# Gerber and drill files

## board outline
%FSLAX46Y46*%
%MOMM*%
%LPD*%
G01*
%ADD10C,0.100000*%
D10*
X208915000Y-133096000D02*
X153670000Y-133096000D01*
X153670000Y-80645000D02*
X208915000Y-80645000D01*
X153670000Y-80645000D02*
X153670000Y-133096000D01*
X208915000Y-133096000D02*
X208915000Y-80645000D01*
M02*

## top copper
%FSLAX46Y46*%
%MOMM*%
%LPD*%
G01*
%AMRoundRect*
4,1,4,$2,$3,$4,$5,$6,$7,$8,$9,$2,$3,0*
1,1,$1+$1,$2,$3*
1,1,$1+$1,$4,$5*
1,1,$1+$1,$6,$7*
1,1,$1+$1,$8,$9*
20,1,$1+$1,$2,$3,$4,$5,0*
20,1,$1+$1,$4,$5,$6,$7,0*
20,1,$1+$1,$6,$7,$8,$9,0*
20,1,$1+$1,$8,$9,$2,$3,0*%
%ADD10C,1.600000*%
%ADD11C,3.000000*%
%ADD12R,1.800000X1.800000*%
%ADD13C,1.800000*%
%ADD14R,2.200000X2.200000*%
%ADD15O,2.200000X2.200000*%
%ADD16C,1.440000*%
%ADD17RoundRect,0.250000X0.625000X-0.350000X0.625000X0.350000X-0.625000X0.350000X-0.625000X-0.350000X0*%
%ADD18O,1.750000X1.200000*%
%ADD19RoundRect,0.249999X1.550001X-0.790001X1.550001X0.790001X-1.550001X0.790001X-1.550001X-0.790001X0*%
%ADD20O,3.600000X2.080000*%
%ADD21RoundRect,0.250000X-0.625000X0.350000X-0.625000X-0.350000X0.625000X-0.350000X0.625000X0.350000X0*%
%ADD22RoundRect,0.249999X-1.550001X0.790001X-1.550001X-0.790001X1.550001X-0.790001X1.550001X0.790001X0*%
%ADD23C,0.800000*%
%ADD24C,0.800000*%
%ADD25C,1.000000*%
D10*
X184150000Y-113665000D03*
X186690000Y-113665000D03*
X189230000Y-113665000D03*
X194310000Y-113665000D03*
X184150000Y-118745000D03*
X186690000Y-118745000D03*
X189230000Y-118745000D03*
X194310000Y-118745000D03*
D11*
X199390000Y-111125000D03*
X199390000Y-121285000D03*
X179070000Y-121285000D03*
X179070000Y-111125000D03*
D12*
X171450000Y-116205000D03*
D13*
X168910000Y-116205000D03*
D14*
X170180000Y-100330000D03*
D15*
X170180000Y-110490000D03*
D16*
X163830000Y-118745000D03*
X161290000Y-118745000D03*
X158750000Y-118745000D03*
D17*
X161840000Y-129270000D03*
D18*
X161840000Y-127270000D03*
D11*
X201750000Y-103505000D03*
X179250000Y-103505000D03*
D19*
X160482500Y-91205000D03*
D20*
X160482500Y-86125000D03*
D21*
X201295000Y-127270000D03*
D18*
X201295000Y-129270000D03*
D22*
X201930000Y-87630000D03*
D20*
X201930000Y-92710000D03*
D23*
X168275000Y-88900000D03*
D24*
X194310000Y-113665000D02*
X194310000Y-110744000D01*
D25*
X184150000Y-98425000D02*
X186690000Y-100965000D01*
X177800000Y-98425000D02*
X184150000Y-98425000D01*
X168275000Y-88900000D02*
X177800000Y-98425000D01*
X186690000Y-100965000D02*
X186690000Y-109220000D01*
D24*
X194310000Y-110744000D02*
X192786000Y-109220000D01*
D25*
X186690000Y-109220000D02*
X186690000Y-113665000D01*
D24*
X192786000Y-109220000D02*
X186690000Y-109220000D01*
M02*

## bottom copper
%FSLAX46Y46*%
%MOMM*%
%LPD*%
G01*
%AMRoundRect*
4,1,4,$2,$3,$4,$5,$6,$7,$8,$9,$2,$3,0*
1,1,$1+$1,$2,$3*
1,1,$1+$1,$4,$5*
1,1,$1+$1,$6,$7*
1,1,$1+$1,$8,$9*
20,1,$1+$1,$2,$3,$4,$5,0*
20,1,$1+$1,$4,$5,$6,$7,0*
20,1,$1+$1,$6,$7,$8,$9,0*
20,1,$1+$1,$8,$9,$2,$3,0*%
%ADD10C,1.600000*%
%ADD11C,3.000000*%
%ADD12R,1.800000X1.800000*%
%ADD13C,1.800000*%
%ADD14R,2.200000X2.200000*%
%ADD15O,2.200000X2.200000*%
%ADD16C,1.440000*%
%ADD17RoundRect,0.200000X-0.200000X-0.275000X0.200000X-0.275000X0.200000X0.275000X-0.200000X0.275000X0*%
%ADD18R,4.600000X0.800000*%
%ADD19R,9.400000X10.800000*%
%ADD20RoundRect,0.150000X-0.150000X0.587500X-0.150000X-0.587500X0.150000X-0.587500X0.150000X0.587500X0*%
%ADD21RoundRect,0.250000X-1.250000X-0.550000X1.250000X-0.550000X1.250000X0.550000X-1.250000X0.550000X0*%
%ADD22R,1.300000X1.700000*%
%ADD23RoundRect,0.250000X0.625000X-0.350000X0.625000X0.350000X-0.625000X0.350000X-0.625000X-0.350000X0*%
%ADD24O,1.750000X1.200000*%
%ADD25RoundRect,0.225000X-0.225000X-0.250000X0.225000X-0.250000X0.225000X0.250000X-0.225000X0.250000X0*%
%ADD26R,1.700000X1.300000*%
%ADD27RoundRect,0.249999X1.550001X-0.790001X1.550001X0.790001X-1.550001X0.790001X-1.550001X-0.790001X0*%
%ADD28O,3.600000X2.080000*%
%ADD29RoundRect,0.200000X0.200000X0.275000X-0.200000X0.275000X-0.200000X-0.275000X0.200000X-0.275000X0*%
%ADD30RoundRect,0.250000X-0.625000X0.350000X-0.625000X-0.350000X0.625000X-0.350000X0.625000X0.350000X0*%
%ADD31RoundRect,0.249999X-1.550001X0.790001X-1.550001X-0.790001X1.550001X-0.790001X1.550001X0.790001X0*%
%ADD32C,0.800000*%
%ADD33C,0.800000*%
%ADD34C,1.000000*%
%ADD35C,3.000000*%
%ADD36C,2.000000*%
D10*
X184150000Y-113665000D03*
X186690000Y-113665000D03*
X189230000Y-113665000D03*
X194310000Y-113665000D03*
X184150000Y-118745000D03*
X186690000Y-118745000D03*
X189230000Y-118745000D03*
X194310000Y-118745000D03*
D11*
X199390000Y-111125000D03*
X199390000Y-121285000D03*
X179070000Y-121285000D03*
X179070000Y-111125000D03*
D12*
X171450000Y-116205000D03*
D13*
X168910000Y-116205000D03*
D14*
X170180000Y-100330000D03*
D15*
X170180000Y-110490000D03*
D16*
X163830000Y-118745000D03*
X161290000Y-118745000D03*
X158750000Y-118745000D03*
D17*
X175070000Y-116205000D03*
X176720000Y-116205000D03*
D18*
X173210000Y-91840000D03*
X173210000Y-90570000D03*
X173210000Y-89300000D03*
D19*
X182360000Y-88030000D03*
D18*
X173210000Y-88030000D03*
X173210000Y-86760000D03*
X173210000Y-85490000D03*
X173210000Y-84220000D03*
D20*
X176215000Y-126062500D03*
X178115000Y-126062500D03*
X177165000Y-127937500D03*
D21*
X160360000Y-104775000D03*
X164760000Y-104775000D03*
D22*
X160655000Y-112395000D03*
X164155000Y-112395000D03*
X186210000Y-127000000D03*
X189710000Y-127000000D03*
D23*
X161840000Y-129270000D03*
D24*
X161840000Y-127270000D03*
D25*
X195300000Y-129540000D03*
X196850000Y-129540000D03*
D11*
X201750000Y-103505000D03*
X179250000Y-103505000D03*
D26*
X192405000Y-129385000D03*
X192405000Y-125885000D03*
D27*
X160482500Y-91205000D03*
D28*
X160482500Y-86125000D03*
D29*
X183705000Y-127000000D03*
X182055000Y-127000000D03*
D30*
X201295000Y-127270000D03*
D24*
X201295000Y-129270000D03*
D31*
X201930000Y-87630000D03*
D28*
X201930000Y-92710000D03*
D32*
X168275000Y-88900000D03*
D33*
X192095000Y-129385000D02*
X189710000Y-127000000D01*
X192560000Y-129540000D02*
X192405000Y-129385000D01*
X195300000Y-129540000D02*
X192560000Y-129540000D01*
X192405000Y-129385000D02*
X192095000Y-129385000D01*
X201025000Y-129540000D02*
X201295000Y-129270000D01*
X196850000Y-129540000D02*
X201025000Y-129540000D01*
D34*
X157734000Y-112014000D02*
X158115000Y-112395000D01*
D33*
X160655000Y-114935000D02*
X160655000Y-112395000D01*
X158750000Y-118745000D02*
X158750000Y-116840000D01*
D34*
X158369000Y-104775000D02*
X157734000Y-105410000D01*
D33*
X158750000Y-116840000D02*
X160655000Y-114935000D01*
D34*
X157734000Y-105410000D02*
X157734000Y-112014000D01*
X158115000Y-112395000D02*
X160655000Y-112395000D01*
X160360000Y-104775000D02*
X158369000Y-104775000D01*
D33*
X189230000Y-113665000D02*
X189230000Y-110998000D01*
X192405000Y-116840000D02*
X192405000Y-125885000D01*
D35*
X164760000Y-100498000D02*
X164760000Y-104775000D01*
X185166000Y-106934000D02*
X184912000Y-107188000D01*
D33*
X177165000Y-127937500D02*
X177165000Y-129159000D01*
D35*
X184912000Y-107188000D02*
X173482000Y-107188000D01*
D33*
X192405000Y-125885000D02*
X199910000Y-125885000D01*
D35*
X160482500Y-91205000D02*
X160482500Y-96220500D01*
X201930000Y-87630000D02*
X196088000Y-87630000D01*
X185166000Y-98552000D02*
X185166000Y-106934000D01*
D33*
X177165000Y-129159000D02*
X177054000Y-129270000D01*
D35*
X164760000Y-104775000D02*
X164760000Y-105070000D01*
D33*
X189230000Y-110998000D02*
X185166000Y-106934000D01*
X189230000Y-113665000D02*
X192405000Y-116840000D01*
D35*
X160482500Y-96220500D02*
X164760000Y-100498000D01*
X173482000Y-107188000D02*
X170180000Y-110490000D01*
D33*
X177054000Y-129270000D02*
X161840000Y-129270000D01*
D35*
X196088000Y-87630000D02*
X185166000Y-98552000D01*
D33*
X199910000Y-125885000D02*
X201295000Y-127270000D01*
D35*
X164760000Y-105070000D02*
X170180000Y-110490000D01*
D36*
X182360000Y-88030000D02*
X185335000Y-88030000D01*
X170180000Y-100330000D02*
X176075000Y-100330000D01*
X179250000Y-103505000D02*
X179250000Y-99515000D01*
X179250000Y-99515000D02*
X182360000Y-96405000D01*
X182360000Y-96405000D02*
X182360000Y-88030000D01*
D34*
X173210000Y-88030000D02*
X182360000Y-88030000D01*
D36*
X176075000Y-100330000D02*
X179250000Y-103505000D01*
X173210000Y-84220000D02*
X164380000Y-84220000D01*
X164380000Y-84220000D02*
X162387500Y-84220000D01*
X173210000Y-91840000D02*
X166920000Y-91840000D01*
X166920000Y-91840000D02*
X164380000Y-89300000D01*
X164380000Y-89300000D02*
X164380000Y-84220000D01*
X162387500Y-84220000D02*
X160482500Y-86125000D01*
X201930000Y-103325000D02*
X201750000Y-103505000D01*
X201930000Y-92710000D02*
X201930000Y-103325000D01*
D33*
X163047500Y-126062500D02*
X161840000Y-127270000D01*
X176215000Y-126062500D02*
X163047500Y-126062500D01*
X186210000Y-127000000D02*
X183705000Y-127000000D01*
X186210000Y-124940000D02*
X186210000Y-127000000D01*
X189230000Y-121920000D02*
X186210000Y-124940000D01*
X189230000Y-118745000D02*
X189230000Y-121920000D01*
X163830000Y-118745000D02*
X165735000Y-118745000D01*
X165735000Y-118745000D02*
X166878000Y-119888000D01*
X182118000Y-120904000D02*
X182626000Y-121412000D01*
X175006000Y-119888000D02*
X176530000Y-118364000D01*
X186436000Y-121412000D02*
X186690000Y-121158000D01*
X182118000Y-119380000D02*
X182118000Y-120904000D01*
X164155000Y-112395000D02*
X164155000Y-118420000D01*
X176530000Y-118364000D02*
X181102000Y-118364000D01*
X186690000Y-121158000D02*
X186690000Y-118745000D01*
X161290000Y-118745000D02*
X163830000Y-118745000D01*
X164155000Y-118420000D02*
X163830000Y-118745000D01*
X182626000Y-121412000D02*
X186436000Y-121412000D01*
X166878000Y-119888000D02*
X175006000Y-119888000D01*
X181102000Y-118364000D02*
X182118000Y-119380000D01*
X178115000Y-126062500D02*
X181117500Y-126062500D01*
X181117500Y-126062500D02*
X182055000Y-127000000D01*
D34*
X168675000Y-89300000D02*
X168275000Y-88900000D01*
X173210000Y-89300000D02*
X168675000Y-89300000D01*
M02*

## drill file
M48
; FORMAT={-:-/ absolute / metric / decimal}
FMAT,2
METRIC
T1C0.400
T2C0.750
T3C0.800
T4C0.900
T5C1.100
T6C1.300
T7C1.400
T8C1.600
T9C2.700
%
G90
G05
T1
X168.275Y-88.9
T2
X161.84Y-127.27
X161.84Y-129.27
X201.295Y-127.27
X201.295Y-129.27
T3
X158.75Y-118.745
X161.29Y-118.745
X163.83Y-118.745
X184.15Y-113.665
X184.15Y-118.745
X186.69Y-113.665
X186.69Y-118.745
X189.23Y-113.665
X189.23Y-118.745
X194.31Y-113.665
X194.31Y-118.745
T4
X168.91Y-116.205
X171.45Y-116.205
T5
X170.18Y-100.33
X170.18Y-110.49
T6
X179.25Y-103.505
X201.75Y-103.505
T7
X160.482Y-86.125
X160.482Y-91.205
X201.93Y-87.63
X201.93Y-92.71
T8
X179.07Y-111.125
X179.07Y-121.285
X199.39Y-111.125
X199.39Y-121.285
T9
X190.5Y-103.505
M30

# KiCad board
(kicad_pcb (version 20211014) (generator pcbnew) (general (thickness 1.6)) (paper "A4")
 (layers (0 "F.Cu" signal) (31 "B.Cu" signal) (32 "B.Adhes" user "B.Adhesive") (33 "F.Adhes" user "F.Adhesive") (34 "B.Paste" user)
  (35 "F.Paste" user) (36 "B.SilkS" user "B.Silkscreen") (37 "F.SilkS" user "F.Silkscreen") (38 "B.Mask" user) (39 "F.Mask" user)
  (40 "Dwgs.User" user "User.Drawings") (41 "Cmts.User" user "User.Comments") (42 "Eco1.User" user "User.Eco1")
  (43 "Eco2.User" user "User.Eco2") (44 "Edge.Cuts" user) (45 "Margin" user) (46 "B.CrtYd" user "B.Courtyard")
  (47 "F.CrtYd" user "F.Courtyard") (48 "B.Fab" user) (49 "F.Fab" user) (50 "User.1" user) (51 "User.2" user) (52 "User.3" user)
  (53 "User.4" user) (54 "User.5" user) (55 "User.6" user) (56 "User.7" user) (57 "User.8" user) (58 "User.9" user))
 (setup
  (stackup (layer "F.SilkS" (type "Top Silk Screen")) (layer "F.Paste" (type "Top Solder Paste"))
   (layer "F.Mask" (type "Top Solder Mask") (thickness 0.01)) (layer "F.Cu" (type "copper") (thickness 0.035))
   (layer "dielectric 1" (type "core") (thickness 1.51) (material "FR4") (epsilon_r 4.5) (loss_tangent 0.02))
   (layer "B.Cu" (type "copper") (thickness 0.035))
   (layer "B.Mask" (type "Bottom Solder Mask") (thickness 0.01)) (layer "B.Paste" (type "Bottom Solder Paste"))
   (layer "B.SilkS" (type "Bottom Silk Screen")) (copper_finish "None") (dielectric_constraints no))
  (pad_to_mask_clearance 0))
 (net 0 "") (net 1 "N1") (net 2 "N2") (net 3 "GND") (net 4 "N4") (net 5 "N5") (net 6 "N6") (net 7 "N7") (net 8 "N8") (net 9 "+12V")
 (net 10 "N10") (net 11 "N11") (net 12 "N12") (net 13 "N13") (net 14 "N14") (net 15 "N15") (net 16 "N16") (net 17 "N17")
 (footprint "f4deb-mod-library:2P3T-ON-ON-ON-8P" (layer "F.Cu") (at 184.15 113.665)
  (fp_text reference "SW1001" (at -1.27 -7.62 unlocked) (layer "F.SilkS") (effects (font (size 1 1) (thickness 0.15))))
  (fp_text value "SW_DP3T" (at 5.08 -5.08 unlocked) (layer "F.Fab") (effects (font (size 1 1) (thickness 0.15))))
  (pad "1" thru_hole circle (at 0 0) (size 1.6 1.6) (drill 0.8) (layers *.Cu *.Mask) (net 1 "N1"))
  (pad "2" thru_hole circle (at 2.54 0) (size 1.6 1.6) (drill 0.8) (layers *.Cu *.Mask) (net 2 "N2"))
  (pad "3" thru_hole circle (at 5.08 0) (size 1.6 1.6) (drill 0.8) (layers *.Cu *.Mask) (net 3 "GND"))
  (pad "4" thru_hole circle (at 10.16 0) (size 1.6 1.6) (drill 0.8) (layers *.Cu *.Mask) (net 2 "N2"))
  (pad "5" thru_hole circle (at 0 5.08) (size 1.6 1.6) (drill 0.8) (layers *.Cu *.Mask) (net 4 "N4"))
  (pad "6" thru_hole circle (at 2.54 5.08) (size 1.6 1.6) (drill 0.8) (layers *.Cu *.Mask) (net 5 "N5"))
  (pad "7" thru_hole circle (at 5.08 5.08) (size 1.6 1.6) (drill 0.8) (layers *.Cu *.Mask) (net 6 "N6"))
  (pad "8" thru_hole circle (at 10.16 5.08) (size 1.6 1.6) (drill 0.8) (layers *.Cu *.Mask) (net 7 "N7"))
  (pad "9" thru_hole circle (at 15.24 -2.54) (size 3 3) (drill 1.6) (layers *.Cu *.Mask))
  (pad "10" thru_hole circle (at 15.24 7.62) (size 3 3) (drill 1.6) (layers *.Cu *.Mask))
  (pad "11" thru_hole circle (at -5.08 7.62) (size 3 3) (drill 1.6) (layers *.Cu *.Mask))
  (pad "12" thru_hole circle (at -5.08 -2.54) (size 3 3) (drill 1.6) (layers *.Cu *.Mask)))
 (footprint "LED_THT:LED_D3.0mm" (layer "F.Cu") (at 171.45 116.205 180)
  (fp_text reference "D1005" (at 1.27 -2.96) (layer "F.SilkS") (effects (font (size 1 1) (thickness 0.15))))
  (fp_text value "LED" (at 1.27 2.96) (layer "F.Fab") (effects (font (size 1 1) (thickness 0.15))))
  (pad "1" thru_hole rect (at 0 0 180) (size 1.8 1.8) (drill 0.9) (layers *.Cu *.Mask) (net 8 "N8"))
  (pad "2" thru_hole circle (at 2.54 0 180) (size 1.8 1.8) (drill 0.9) (layers *.Cu *.Mask) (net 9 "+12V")))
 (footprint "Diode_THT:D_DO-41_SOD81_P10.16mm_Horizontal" (layer "B.Cu") (at 170.18 100.33 -90)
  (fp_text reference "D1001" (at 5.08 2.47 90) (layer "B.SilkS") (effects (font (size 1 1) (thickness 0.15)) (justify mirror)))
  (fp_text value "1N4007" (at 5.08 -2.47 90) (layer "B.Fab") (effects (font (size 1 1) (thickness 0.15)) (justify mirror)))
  (pad "1" thru_hole rect (at 0 0 270) (size 2.2 2.2) (drill 1.1) (layers *.Cu *.Mask) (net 9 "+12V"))
  (pad "2" thru_hole oval (at 10.16 0 270) (size 2.2 2.2) (drill 1.1) (layers *.Cu *.Mask) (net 3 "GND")))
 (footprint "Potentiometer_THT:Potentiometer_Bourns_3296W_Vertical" (layer "B.Cu") (at 163.83 118.745)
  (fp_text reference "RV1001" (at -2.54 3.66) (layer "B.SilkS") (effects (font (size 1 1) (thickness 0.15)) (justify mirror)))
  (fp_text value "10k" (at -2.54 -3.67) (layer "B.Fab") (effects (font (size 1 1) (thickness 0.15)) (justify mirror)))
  (pad "1" thru_hole circle (at 0 0) (size 1.44 1.44) (drill 0.8) (layers *.Cu *.Mask) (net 5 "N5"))
  (pad "2" thru_hole circle (at -2.54 0) (size 1.44 1.44) (drill 0.8) (layers *.Cu *.Mask) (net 5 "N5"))
  (pad "3" thru_hole circle (at -5.08 0) (size 1.44 1.44) (drill 0.8) (layers *.Cu *.Mask) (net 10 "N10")))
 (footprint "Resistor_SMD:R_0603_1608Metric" (layer "B.Cu") (at 175.895 116.205)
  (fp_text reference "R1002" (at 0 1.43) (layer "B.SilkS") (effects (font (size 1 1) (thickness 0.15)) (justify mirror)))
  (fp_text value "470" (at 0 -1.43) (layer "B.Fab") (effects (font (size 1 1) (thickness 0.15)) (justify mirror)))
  (pad "1" smd roundrect (at -0.825 0) (size 0.8 0.95) (layers "B.Cu" "B.Paste" "B.Mask") (roundrect_rratio 0.25) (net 8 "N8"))
  (pad "2" smd roundrect (at 0.825 0) (size 0.8 0.95) (layers "B.Cu" "B.Paste" "B.Mask") (roundrect_rratio 0.25) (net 3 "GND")))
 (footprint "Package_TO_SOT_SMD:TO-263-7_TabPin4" (layer "B.Cu") (at 178.985 88.03)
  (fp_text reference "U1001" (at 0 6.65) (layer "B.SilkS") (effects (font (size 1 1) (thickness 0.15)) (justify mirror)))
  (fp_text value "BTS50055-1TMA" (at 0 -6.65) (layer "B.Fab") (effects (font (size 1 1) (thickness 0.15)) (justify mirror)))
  (pad "" smd rect (at 0.95 -2.775) (size 4.55 5.25) (layers "B.Paste"))
  (pad "" smd rect (at 0.95 2.775) (size 4.55 5.25) (layers "B.Paste"))
  (pad "" smd rect (at 5.8 2.775) (size 4.55 5.25) (layers "B.Paste"))
  (pad "" smd rect (at 5.8 -2.775) (size 4.55 5.25) (layers "B.Paste"))
  (pad "1" smd rect (at -5.775 3.81) (size 4.6 0.8) (layers "B.Cu" "B.Paste" "B.Mask") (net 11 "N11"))
  (pad "2" smd rect (at -5.775 2.54) (size 4.6 0.8) (layers "B.Cu" "B.Paste" "B.Mask") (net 11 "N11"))
  (pad "3" smd rect (at -5.775 1.27) (size 4.6 0.8) (layers "B.Cu" "B.Paste" "B.Mask") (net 2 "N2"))
  (pad "4" smd rect (at 3.375 0) (size 9.4 10.8) (layers "B.Cu" "B.Mask") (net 9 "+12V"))
  (pad "4" smd rect (at -5.775 0) (size 4.6 0.8) (layers "B.Cu" "B.Paste" "B.Mask") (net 9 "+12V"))
  (pad "5" smd rect (at -5.775 -1.27) (size 4.6 0.8) (layers "B.Cu" "B.Paste" "B.Mask") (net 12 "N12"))
  (pad "6" smd rect (at -5.775 -2.54) (size 4.6 0.8) (layers "B.Cu" "B.Paste" "B.Mask") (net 11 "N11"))
  (pad "7" smd rect (at -5.775 -3.81) (size 4.6 0.8) (layers "B.Cu" "B.Paste" "B.Mask") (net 11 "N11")))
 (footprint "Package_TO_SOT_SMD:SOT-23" (layer "B.Cu") (at 177.165 127 -90)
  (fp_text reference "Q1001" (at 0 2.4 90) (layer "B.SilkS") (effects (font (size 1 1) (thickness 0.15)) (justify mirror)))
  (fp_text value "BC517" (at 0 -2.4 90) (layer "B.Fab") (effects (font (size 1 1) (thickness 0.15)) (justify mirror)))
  (pad "1" smd roundrect (at -0.9375 0.95 270) (size 1.475 0.6) (layers "B.Cu" "B.Paste" "B.Mask") (roundrect_rratio 0.25) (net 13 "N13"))
  (pad "2" smd roundrect (at -0.9375 -0.95 270) (size 1.475 0.6) (layers "B.Cu" "B.Paste" "B.Mask") (roundrect_rratio 0.25) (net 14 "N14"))
  (pad "3" smd roundrect (at 0.9375 0 270) (size 1.475 0.6) (layers "B.Cu" "B.Paste" "B.Mask") (roundrect_rratio 0.25) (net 3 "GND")))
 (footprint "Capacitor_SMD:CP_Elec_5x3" (layer "B.Cu") (at 162.56 104.775)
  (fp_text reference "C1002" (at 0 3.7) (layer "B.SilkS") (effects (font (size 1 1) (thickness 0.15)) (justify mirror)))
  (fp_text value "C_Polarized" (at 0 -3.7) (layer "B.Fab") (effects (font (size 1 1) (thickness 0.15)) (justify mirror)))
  (pad "1" smd roundrect (at -2.2 0) (size 3 1.6) (layers "B.Cu" "B.Paste" "B.Mask") (roundrect_rratio 0.15625) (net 10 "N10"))
  (pad "2" smd roundrect (at 2.2 0) (size 3 1.6) (layers "B.Cu" "B.Paste" "B.Mask") (roundrect_rratio 0.15625) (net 3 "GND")))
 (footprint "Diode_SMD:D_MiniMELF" (layer "B.Cu") (at 162.405 112.395)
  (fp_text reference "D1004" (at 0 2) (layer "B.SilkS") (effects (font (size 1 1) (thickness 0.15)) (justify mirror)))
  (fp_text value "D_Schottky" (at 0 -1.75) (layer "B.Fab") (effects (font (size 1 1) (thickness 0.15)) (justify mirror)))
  (pad "1" smd rect (at -1.75 0) (size 1.3 1.7) (layers "B.Cu" "B.Paste" "B.Mask") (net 10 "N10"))
  (pad "2" smd rect (at 1.75 0) (size 1.3 1.7) (layers "B.Cu" "B.Paste" "B.Mask") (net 5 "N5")))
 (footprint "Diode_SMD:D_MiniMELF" (layer "B.Cu") (at 187.96 127)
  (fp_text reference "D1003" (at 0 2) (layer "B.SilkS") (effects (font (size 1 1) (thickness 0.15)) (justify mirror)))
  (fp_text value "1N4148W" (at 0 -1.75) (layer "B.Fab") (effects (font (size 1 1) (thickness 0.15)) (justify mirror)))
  (pad "1" smd rect (at -1.75 0) (size 1.3 1.7) (layers "B.Cu" "B.Paste" "B.Mask") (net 6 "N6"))
  (pad "2" smd rect (at 1.75 0) (size 1.3 1.7) (layers "B.Cu" "B.Paste" "B.Mask") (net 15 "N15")))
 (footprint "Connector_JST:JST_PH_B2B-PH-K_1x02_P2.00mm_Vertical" (layer "B.Cu") (at 161.84 129.27 90)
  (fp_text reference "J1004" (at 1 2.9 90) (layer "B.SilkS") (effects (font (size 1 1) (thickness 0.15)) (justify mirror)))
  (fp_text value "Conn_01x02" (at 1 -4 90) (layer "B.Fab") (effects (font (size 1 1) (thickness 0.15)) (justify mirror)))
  (pad "1" thru_hole roundrect (at 0 0 90) (size 1.2 1.75) (drill 0.75) (layers *.Cu *.Mask) (roundrect_rratio 0.208333) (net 3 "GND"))
  (pad "2" thru_hole oval (at 2 0 90) (size 1.2 1.75) (drill 0.75) (layers *.Cu *.Mask) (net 13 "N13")))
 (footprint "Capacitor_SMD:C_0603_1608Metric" (layer "B.Cu") (at 196.075 129.54)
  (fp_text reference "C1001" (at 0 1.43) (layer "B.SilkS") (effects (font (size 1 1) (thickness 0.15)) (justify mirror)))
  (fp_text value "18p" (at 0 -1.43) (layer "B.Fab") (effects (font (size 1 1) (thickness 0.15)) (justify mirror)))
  (pad "1" smd roundrect (at -0.775 0) (size 0.9 0.95) (layers "B.Cu" "B.Paste" "B.Mask") (roundrect_rratio 0.25) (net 15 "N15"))
  (pad "2" smd roundrect (at 0.775 0) (size 0.9 0.95) (layers "B.Cu" "B.Paste" "B.Mask") (roundrect_rratio 0.25) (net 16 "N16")))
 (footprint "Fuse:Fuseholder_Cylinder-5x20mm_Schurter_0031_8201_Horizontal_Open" (layer "B.Cu") (at 201.75 103.505 180)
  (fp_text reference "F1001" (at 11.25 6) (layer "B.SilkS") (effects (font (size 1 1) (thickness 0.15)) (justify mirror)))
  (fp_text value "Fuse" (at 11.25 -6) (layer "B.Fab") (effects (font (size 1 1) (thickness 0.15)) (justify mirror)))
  (pad "" np_thru_hole circle (at 11.25 0 180) (size 2.7 2.7) (drill 2.7) (layers *.Cu *.Mask))
  (pad "1" thru_hole circle (at 0 0 180) (size 3 3) (drill 1.3) (layers *.Cu *.Mask) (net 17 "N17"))
  (pad "2" thru_hole circle (at 22.5 0 180) (size 3 3) (drill 1.3) (layers *.Cu *.Mask) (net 9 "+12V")))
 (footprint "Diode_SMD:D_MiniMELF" (layer "B.Cu") (at 192.405 127.635 90)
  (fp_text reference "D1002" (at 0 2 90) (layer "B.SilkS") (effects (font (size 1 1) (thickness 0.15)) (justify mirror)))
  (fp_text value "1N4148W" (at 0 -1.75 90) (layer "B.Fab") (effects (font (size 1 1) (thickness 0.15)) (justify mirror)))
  (pad "1" smd rect (at -1.75 0 90) (size 1.3 1.7) (layers "B.Cu" "B.Paste" "B.Mask") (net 15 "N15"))
  (pad "2" smd rect (at 1.75 0 90) (size 1.3 1.7) (layers "B.Cu" "B.Paste" "B.Mask") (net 3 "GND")))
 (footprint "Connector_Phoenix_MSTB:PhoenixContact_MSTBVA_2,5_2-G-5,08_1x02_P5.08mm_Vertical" (layer "B.Cu") (at 160.4825 91.205 90)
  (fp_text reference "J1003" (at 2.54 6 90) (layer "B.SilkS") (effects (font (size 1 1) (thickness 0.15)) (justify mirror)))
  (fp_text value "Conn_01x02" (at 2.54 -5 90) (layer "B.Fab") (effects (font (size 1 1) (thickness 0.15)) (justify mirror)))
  (pad "1" thru_hole roundrect (at 0 0 90) (size 2.08 3.6) (drill 1.4) (layers *.Cu *.Mask) (roundrect_rratio 0.120192) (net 3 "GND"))
  (pad "2" thru_hole oval (at 5.08 0 90) (size 2.08 3.6) (drill 1.4) (layers *.Cu *.Mask) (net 11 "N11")))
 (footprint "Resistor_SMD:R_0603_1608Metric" (layer "B.Cu") (at 182.88 127 180)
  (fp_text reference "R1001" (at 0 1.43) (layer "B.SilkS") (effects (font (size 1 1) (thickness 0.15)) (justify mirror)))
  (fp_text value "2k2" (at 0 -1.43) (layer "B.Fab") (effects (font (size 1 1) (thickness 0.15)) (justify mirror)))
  (pad "1" smd roundrect (at -0.825 0 180) (size 0.8 0.95) (layers "B.Cu" "B.Paste" "B.Mask") (roundrect_rratio 0.25) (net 6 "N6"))
  (pad "2" smd roundrect (at 0.825 0 180) (size 0.8 0.95) (layers "B.Cu" "B.Paste" "B.Mask") (roundrect_rratio 0.25) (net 14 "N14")))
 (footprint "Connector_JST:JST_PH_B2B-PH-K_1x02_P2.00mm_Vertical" (layer "B.Cu") (at 201.295 127.27 -90)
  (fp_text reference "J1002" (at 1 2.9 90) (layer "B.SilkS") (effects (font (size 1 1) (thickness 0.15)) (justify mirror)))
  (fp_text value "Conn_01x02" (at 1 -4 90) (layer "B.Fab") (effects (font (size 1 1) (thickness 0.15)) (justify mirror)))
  (pad "1" thru_hole roundrect (at 0 0 270) (size 1.2 1.75) (drill 0.75) (layers *.Cu *.Mask) (roundrect_rratio 0.208333) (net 3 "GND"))
  (pad "2" thru_hole oval (at 2 0 270) (size 1.2 1.75) (drill 0.75) (layers *.Cu *.Mask) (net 16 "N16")))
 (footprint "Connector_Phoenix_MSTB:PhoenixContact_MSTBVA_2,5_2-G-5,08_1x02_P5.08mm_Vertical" (layer "B.Cu") (at 201.93 87.63 -90)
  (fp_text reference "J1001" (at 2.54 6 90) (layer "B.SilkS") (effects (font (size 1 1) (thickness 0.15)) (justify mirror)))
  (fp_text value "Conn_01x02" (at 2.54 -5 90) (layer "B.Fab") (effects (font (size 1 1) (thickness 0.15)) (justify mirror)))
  (pad "1" thru_hole roundrect (at 0 0 270) (size 2.08 3.6) (drill 1.4) (layers *.Cu *.Mask) (roundrect_rratio 0.120192) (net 3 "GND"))
  (pad "2" thru_hole oval (at 5.08 0 270) (size 2.08 3.6) (drill 1.4) (layers *.Cu *.Mask) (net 17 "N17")))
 (gr_line (start 208.915 133.096) (end 153.67 133.096) (layer "Edge.Cuts") (width 0.1))
 (gr_line (start 153.67 80.645) (end 208.915 80.645) (layer "Edge.Cuts") (width 0.1))
 (gr_line (start 153.67 80.645) (end 153.67 133.096) (layer "Edge.Cuts") (width 0.1))
 (gr_line (start 208.915 133.096) (end 208.915 80.645) (layer "Edge.Cuts") (width 0.1))
 (segment (start 192.095 129.385) (end 189.71 127) (width 0.8) (layer "B.Cu") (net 15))
 (segment (start 192.56 129.54) (end 192.405 129.385) (width 0.8) (layer "B.Cu") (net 15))
 (segment (start 195.3 129.54) (end 192.56 129.54) (width 0.8) (layer "B.Cu") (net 15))
 (segment (start 192.405 129.385) (end 192.095 129.385) (width 0.8) (layer "B.Cu") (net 15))
 (segment (start 201.025 129.54) (end 201.295 129.27) (width 0.8) (layer "B.Cu") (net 16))
 (segment (start 196.85 129.54) (end 201.025 129.54) (width 0.8) (layer "B.Cu") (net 16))
 (segment (start 157.734 112.014) (end 158.115 112.395) (width 1) (layer "B.Cu") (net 10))
 (segment (start 160.655 114.935) (end 160.655 112.395) (width 0.8) (layer "B.Cu") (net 10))
 (segment (start 158.75 118.745) (end 158.75 116.84) (width 0.8) (layer "B.Cu") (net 10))
 (segment (start 158.369 104.775) (end 157.734 105.41) (width 1) (layer "B.Cu") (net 10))
 (segment (start 158.75 116.84) (end 160.655 114.935) (width 0.8) (layer "B.Cu") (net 10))
 (segment (start 157.734 105.41) (end 157.734 112.014) (width 1) (layer "B.Cu") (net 10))
 (segment (start 158.115 112.395) (end 160.655 112.395) (width 1) (layer "B.Cu") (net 10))
 (segment (start 160.36 104.775) (end 158.369 104.775) (width 1) (layer "B.Cu") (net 10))
 (segment (start 189.23 113.665) (end 189.23 110.998) (width 0.8) (layer "B.Cu") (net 3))
 (segment (start 192.405 116.84) (end 192.405 125.885) (width 0.8) (layer "B.Cu") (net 3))
 (segment (start 164.76 100.498) (end 164.76 104.775) (width 3) (layer "B.Cu") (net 3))
 (segment (start 185.166 106.934) (end 184.912 107.188) (width 3) (layer "B.Cu") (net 3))
 (segment (start 177.165 127.9375) (end 177.165 129.159) (width 0.8) (layer "B.Cu") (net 3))
 (segment (start 184.912 107.188) (end 173.482 107.188) (width 3) (layer "B.Cu") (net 3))
 (segment (start 192.405 125.885) (end 199.91 125.885) (width 0.8) (layer "B.Cu") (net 3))
 (segment (start 160.4825 91.205) (end 160.4825 96.2205) (width 3) (layer "B.Cu") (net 3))
 (segment (start 201.93 87.63) (end 196.088 87.63) (width 3) (layer "B.Cu") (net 3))
 (segment (start 185.166 98.552) (end 185.166 106.934) (width 3) (layer "B.Cu") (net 3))
 (segment (start 177.165 129.159) (end 177.054 129.27) (width 0.8) (layer "B.Cu") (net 3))
 (segment (start 164.76 104.775) (end 164.76 105.07) (width 3) (layer "B.Cu") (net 3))
 (segment (start 189.23 110.998) (end 185.166 106.934) (width 0.8) (layer "B.Cu") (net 3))
 (segment (start 189.23 113.665) (end 192.405 116.84) (width 0.8) (layer "B.Cu") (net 3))
 (segment (start 160.4825 96.2205) (end 164.76 100.498) (width 3) (layer "B.Cu") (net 3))
 (segment (start 173.482 107.188) (end 170.18 110.49) (width 3) (layer "B.Cu") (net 3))
 (segment (start 177.054 129.27) (end 161.84 129.27) (width 0.8) (layer "B.Cu") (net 3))
 (segment (start 196.088 87.63) (end 185.166 98.552) (width 3) (layer "B.Cu") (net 3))
 (segment (start 199.91 125.885) (end 201.295 127.27) (width 0.8) (layer "B.Cu") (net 3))
 (segment (start 164.76 105.07) (end 170.18 110.49) (width 3) (layer "B.Cu") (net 3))
 (segment (start 182.36 88.03) (end 185.335 88.03) (width 2) (layer "B.Cu") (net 9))
 (segment (start 170.18 100.33) (end 176.075 100.33) (width 2) (layer "B.Cu") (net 9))
 (segment (start 179.25 103.505) (end 179.25 99.515) (width 2) (layer "B.Cu") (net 9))
 (segment (start 179.25 99.515) (end 182.36 96.405) (width 2) (layer "B.Cu") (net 9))
 (segment (start 182.36 96.405) (end 182.36 88.03) (width 2) (layer "B.Cu") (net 9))
 (segment (start 173.21 88.03) (end 182.36 88.03) (width 1) (layer "B.Cu") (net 9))
 (segment (start 176.075 100.33) (end 179.25 103.505) (width 2) (layer "B.Cu") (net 9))
 (segment (start 173.21 84.22) (end 164.38 84.22) (width 2) (layer "B.Cu") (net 11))
 (segment (start 164.38 84.22) (end 162.3875 84.22) (width 2) (layer "B.Cu") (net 11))
 (segment (start 173.21 91.84) (end 166.92 91.84) (width 2) (layer "B.Cu") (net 11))
 (segment (start 166.92 91.84) (end 164.38 89.3) (width 2) (layer "B.Cu") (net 11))
 (segment (start 164.38 89.3) (end 164.38 84.22) (width 2) (layer "B.Cu") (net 11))
 (segment (start 162.3875 84.22) (end 160.4825 86.125) (width 2) (layer "B.Cu") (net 11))
 (segment (start 201.93 103.325) (end 201.75 103.505) (width 2) (layer "B.Cu") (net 17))
 (segment (start 201.93 92.71) (end 201.93 103.325) (width 2) (layer "B.Cu") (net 17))
 (segment (start 163.0475 126.0625) (end 161.84 127.27) (width 0.8) (layer "B.Cu") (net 13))
 (segment (start 176.215 126.0625) (end 163.0475 126.0625) (width 0.8) (layer "B.Cu") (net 13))
 (segment (start 186.21 127) (end 183.705 127) (width 0.8) (layer "B.Cu") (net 6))
 (segment (start 186.21 124.94) (end 186.21 127) (width 0.8) (layer "B.Cu") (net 6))
 (segment (start 189.23 121.92) (end 186.21 124.94) (width 0.8) (layer "B.Cu") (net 6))
 (segment (start 189.23 118.745) (end 189.23 121.92) (width 0.8) (layer "B.Cu") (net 6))
 (segment (start 163.83 118.745) (end 165.735 118.745) (width 0.8) (layer "B.Cu") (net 5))
 (segment (start 165.735 118.745) (end 166.878 119.888) (width 0.8) (layer "B.Cu") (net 5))
 (segment (start 182.118 120.904) (end 182.626 121.412) (width 0.8) (layer "B.Cu") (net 5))
 (segment (start 175.006 119.888) (end 176.53 118.364) (width 0.8) (layer "B.Cu") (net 5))
 (segment (start 186.436 121.412) (end 186.69 121.158) (width 0.8) (layer "B.Cu") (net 5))
 (segment (start 182.118 119.38) (end 182.118 120.904) (width 0.8) (layer "B.Cu") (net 5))
 (segment (start 164.155 112.395) (end 164.155 118.42) (width 0.8) (layer "B.Cu") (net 5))
 (segment (start 176.53 118.364) (end 181.102 118.364) (width 0.8) (layer "B.Cu") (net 5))
 (segment (start 186.69 121.158) (end 186.69 118.745) (width 0.8) (layer "B.Cu") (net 5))
 (segment (start 161.29 118.745) (end 163.83 118.745) (width 0.8) (layer "B.Cu") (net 5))
 (segment (start 164.155 118.42) (end 163.83 118.745) (width 0.8) (layer "B.Cu") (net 5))
 (segment (start 182.626 121.412) (end 186.436 121.412) (width 0.8) (layer "B.Cu") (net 5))
 (segment (start 166.878 119.888) (end 175.006 119.888) (width 0.8) (layer "B.Cu") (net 5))
 (segment (start 181.102 118.364) (end 182.118 119.38) (width 0.8) (layer "B.Cu") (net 5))
 (segment (start 178.115 126.0625) (end 181.1175 126.0625) (width 0.8) (layer "B.Cu") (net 14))
 (segment (start 181.1175 126.0625) (end 182.055 127) (width 0.8) (layer "B.Cu") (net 14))
 (segment (start 194.31 113.665) (end 194.31 110.744) (width 0.8) (layer "F.Cu") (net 2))
 (segment (start 184.15 98.425) (end 186.69 100.965) (width 1) (layer "F.Cu") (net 2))
 (segment (start 177.8 98.425) (end 184.15 98.425) (width 1) (layer "F.Cu") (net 2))
 (segment (start 168.275 88.9) (end 177.8 98.425) (width 1) (layer "F.Cu") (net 2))
 (segment (start 186.69 100.965) (end 186.69 109.22) (width 1) (layer "F.Cu") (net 2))
 (segment (start 194.31 110.744) (end 192.786 109.22) (width 0.8) (layer "F.Cu") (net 2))
 (segment (start 186.69 109.22) (end 186.69 113.665) (width 1) (layer "F.Cu") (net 2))
 (segment (start 192.786 109.22) (end 186.69 109.22) (width 0.8) (layer "F.Cu") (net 2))
 (via (at 168.275 88.9) (size 0.8) (drill 0.4) (layers "F.Cu" "B.Cu") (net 2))
 (segment (start 168.675 89.3) (end 168.275 88.9) (width 1) (layer "B.Cu") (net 2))
 (segment (start 173.21 89.3) (end 168.675 89.3) (width 1) (layer "B.Cu") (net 2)))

